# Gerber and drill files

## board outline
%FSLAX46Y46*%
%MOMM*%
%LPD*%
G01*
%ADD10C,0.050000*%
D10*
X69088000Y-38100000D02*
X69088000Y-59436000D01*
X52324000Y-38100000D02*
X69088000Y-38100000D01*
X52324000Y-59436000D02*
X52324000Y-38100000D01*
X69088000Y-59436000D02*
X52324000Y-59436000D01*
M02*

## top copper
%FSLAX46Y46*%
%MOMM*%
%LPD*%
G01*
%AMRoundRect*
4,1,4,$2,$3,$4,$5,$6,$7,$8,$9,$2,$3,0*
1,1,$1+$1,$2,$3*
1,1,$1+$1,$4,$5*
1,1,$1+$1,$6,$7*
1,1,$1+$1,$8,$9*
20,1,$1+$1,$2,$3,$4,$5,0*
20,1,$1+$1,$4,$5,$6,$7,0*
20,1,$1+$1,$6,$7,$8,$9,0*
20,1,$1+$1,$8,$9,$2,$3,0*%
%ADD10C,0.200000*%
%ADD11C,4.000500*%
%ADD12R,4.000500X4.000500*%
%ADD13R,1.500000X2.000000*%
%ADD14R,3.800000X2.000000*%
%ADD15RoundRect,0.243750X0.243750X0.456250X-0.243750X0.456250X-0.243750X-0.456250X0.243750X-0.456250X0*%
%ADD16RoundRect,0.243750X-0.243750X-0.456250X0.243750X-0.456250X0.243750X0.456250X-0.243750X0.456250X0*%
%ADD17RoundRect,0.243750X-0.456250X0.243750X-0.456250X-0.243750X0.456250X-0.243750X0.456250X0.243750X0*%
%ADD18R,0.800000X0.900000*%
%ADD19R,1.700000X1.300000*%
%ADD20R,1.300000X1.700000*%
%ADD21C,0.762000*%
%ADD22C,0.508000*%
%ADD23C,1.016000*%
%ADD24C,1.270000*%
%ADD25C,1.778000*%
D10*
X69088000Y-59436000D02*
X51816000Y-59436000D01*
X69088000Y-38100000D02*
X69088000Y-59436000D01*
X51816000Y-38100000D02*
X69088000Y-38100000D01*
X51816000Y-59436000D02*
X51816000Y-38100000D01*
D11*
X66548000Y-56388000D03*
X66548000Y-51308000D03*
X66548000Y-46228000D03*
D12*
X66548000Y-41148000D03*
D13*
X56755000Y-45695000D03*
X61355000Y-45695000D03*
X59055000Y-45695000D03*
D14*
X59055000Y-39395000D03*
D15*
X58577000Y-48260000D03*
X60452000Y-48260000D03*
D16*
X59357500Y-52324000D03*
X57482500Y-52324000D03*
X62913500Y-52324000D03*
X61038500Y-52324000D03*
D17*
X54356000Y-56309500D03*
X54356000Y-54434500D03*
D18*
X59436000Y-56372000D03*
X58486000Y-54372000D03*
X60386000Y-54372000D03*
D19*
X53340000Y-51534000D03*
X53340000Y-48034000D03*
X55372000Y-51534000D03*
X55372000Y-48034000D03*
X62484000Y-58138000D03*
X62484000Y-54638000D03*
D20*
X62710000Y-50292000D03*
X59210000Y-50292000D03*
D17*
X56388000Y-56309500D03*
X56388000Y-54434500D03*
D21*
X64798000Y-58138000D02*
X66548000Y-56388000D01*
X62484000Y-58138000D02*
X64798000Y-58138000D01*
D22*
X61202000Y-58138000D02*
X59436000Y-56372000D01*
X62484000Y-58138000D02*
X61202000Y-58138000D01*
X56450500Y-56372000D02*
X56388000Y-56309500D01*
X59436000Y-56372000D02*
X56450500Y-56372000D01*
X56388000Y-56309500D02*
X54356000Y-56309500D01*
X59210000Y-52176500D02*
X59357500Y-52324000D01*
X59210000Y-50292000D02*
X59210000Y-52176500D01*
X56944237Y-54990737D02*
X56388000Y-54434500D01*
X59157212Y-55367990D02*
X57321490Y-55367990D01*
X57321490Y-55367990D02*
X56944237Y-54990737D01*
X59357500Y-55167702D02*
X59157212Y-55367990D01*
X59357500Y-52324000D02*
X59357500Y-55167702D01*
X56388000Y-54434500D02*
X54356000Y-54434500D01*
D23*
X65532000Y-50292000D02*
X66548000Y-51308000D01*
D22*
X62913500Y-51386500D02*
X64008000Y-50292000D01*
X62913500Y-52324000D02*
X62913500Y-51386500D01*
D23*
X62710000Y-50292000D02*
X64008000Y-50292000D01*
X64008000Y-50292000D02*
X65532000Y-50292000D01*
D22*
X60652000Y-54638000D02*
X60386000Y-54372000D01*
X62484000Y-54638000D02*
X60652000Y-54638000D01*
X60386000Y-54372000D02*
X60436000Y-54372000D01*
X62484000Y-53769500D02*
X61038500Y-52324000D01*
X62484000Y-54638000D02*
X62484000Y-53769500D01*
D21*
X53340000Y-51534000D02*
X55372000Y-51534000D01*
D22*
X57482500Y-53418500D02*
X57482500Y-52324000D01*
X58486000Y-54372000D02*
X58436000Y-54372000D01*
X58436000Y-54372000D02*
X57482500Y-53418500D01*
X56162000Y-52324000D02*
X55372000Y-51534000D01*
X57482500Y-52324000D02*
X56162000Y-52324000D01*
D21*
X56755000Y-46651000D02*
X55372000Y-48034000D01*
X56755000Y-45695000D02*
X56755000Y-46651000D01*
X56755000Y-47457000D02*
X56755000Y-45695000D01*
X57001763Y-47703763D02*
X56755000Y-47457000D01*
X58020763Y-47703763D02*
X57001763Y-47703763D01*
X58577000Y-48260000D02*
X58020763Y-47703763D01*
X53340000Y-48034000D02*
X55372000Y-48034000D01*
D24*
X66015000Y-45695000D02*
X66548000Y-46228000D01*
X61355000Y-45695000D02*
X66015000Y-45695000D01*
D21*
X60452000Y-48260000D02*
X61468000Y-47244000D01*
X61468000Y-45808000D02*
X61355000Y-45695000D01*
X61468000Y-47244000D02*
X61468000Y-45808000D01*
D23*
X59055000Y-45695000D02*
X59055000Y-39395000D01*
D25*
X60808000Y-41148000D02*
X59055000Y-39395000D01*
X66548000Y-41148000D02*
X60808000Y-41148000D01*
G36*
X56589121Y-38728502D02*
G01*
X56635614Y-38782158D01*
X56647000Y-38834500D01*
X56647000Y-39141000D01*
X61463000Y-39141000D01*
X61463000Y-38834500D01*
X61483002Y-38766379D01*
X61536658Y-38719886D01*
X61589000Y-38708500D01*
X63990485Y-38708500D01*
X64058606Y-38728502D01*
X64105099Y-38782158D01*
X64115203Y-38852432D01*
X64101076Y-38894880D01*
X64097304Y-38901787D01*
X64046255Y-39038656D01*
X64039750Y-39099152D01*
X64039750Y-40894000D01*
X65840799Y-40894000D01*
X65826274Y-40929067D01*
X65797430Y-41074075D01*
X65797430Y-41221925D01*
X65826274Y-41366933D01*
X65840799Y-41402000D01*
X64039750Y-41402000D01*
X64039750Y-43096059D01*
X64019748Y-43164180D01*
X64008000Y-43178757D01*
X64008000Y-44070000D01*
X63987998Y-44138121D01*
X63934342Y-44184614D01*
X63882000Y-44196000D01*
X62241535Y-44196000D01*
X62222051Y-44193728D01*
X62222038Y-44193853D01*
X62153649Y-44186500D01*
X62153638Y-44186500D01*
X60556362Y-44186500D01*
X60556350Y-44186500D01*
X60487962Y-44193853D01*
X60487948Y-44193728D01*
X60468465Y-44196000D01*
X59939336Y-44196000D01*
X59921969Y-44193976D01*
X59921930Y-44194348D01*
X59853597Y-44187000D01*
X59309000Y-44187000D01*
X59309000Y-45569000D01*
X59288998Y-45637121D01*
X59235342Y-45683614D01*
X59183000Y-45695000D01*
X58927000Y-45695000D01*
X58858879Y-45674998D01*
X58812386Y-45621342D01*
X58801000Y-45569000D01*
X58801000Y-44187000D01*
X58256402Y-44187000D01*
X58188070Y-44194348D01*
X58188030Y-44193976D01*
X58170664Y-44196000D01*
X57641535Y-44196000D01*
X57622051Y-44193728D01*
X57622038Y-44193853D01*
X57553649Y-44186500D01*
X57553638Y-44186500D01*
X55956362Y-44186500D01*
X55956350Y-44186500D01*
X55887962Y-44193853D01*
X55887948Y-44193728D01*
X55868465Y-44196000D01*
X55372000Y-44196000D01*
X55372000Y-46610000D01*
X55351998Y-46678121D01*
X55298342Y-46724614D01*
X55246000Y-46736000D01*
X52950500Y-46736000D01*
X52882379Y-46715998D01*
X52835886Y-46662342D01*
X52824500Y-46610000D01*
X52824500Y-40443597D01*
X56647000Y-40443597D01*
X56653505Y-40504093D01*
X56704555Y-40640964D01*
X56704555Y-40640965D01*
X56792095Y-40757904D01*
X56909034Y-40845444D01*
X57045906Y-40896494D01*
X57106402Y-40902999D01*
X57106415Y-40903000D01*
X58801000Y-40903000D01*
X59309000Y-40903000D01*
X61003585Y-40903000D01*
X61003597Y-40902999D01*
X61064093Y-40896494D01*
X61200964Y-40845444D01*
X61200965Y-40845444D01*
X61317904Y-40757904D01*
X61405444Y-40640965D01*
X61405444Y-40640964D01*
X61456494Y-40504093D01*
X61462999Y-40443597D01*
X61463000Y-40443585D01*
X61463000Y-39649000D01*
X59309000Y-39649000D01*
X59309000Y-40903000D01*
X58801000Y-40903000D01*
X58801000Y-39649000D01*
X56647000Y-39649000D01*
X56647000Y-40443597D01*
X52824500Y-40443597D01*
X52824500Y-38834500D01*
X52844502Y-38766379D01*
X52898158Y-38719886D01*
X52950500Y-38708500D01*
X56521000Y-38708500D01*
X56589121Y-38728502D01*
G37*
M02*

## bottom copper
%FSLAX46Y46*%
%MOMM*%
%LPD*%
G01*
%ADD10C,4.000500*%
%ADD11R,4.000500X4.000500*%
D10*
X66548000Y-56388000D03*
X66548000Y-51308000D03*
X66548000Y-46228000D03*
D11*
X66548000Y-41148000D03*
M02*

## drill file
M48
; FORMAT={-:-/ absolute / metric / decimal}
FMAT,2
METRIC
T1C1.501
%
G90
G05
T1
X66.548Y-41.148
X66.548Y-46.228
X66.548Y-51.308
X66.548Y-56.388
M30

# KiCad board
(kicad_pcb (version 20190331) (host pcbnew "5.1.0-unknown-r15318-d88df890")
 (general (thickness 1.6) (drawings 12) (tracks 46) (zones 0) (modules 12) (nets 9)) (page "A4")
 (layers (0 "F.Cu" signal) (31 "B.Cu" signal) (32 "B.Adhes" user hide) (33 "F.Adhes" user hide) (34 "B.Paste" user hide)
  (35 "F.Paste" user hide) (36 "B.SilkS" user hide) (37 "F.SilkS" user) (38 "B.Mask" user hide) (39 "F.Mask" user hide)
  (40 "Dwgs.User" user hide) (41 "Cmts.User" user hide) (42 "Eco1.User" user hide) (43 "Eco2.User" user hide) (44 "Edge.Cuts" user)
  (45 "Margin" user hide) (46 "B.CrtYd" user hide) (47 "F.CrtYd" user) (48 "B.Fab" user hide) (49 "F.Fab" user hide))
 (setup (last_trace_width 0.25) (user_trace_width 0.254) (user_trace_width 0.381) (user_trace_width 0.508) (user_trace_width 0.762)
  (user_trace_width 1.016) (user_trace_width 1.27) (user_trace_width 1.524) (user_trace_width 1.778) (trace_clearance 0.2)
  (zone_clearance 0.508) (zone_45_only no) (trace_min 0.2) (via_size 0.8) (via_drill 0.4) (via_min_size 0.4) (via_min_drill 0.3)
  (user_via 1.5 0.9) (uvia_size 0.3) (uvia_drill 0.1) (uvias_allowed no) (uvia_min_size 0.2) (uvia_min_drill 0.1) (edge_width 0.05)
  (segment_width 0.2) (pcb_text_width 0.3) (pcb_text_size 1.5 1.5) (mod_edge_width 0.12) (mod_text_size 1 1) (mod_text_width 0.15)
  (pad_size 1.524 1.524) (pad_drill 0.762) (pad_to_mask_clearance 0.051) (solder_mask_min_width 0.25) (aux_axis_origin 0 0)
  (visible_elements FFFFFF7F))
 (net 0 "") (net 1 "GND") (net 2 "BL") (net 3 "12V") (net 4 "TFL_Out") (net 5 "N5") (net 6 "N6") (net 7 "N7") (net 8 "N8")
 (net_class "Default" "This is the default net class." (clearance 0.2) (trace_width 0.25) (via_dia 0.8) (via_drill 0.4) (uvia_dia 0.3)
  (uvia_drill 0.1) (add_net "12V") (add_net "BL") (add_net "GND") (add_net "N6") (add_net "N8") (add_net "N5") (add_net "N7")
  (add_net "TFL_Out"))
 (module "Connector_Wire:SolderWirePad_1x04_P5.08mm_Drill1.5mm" (layer "F.Cu") (at 66.548 41.148 270)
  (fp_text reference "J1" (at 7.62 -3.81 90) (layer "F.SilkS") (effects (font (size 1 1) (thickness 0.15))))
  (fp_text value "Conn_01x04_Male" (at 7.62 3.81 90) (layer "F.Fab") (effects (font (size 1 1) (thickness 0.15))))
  (pad "4" thru_hole circle (at 15.24 0 270) (size 4.0005 4.0005) (drill 1.50114) (layers *.Cu *.Mask) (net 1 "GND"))
  (pad "3" thru_hole circle (at 10.16 0 270) (size 4.0005 4.0005) (drill 1.50114) (layers *.Cu *.Mask) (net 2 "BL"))
  (pad "2" thru_hole circle (at 5.08 0 270) (size 4.0005 4.0005) (drill 1.50114) (layers *.Cu *.Mask) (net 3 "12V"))
  (pad "1" thru_hole rect (at 0 0 270) (size 4.0005 4.0005) (drill 1.50114) (layers *.Cu *.Mask) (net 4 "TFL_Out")))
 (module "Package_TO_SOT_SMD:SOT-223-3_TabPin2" (layer "F.Cu") (at 59.055 42.545 90)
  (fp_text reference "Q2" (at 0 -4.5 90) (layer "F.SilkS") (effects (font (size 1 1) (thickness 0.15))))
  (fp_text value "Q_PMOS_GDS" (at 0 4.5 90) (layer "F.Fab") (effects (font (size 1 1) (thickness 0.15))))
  (pad "1" smd rect (at -3.15 -2.3 90) (size 2 1.5) (layers "F.Cu" "F.Paste" "F.Mask") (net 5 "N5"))
  (pad "3" smd rect (at -3.15 2.3 90) (size 2 1.5) (layers "F.Cu" "F.Paste" "F.Mask") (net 3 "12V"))
  (pad "2" smd rect (at -3.15 0 90) (size 2 1.5) (layers "F.Cu" "F.Paste" "F.Mask") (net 4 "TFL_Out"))
  (pad "2" smd rect (at 3.15 0 90) (size 2 3.8) (layers "F.Cu" "F.Paste" "F.Mask") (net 4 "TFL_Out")))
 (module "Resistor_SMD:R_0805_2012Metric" (layer "F.Cu") (at 59.5145 48.26 180)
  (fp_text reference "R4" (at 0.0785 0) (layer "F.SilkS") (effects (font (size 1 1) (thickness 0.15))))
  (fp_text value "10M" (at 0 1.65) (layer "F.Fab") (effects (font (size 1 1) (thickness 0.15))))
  (pad "2" smd roundrect (at 0.9375 0 180) (size 0.975 1.4) (layers "F.Cu" "F.Paste" "F.Mask") (roundrect_rratio 0.25) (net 5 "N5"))
  (pad "1" smd roundrect (at -0.9375 0 180) (size 0.975 1.4) (layers "F.Cu" "F.Paste" "F.Mask") (roundrect_rratio 0.25) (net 3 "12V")))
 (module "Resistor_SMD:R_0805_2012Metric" (layer "F.Cu") (at 58.42 52.324)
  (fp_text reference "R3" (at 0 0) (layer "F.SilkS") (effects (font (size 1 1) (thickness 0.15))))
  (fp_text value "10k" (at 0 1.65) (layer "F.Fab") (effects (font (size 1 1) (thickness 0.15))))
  (pad "2" smd roundrect (at 0.9375 0) (size 0.975 1.4) (layers "F.Cu" "F.Paste" "F.Mask") (roundrect_rratio 0.25) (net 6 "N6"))
  (pad "1" smd roundrect (at -0.9375 0) (size 0.975 1.4) (layers "F.Cu" "F.Paste" "F.Mask") (roundrect_rratio 0.25) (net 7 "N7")))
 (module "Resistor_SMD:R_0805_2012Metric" (layer "F.Cu") (at 61.976 52.324)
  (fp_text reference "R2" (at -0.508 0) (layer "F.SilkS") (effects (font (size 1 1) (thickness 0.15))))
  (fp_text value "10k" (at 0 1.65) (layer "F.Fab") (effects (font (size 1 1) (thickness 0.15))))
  (pad "2" smd roundrect (at 0.9375 0) (size 0.975 1.4) (layers "F.Cu" "F.Paste" "F.Mask") (roundrect_rratio 0.25) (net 2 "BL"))
  (pad "1" smd roundrect (at -0.9375 0) (size 0.975 1.4) (layers "F.Cu" "F.Paste" "F.Mask") (roundrect_rratio 0.25) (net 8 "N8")))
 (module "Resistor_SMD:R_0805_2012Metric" (layer "F.Cu") (at 54.356 55.372 270)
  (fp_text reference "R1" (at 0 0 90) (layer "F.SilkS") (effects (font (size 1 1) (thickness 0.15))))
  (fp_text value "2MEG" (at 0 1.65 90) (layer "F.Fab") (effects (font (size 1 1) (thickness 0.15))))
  (pad "2" smd roundrect (at 0.9375 0 270) (size 0.975 1.4) (layers "F.Cu" "F.Paste" "F.Mask") (roundrect_rratio 0.25) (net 1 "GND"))
  (pad "1" smd roundrect (at -0.9375 0 270) (size 0.975 1.4) (layers "F.Cu" "F.Paste" "F.Mask") (roundrect_rratio 0.25) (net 6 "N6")))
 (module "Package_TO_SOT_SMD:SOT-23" (layer "F.Cu") (at 59.436 55.372 270)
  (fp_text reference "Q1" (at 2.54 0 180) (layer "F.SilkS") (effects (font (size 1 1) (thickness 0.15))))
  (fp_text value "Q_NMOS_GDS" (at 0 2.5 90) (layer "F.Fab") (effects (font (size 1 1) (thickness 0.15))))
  (pad "3" smd rect (at 1 0 270) (size 0.9 0.8) (layers "F.Cu" "F.Paste" "F.Mask") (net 1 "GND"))
  (pad "2" smd rect (at -1 0.95 270) (size 0.9 0.8) (layers "F.Cu" "F.Paste" "F.Mask") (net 7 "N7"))
  (pad "1" smd rect (at -1 -0.95 270) (size 0.9 0.8) (layers "F.Cu" "F.Paste" "F.Mask") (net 8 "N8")))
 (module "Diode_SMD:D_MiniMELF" (layer "F.Cu") (at 53.34 49.784 270)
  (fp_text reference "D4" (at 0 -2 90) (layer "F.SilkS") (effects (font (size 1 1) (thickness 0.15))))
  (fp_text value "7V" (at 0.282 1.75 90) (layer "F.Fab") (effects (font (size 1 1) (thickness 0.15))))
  (pad "2" smd rect (at 1.75 0 270) (size 1.3 1.7) (layers "F.Cu" "F.Paste" "F.Mask") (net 7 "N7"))
  (pad "1" smd rect (at -1.75 0 270) (size 1.3 1.7) (layers "F.Cu" "F.Paste" "F.Mask") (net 5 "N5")))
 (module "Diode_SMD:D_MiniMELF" (layer "F.Cu") (at 55.372 49.784 270)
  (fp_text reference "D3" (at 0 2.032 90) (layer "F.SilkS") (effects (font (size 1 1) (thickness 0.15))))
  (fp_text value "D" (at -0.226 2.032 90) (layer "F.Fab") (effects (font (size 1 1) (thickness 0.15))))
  (pad "2" smd rect (at 1.75 0 270) (size 1.3 1.7) (layers "F.Cu" "F.Paste" "F.Mask") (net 7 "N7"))
  (pad "1" smd rect (at -1.75 0 270) (size 1.3 1.7) (layers "F.Cu" "F.Paste" "F.Mask") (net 5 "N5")))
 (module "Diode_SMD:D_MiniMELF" (layer "F.Cu") (at 62.484 56.388 270)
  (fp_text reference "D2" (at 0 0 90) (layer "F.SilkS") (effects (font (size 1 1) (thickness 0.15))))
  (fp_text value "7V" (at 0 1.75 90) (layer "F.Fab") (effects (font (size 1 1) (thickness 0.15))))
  (pad "2" smd rect (at 1.75 0 270) (size 1.3 1.7) (layers "F.Cu" "F.Paste" "F.Mask") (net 1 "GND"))
  (pad "1" smd rect (at -1.75 0 270) (size 1.3 1.7) (layers "F.Cu" "F.Paste" "F.Mask") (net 8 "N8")))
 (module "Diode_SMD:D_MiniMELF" (layer "F.Cu") (at 60.96 50.292)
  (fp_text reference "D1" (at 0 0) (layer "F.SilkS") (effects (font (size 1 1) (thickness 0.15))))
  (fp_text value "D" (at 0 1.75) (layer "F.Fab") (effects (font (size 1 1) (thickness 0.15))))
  (pad "2" smd rect (at 1.75 0) (size 1.3 1.7) (layers "F.Cu" "F.Paste" "F.Mask") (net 2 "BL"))
  (pad "1" smd rect (at -1.75 0) (size 1.3 1.7) (layers "F.Cu" "F.Paste" "F.Mask") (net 6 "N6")))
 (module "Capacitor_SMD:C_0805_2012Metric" (layer "F.Cu") (at 56.388 55.372 270)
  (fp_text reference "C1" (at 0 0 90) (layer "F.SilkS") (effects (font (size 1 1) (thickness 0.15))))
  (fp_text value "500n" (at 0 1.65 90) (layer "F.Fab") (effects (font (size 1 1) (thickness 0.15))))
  (pad "2" smd roundrect (at 0.9375 0 270) (size 0.975 1.4) (layers "F.Cu" "F.Paste" "F.Mask") (roundrect_rratio 0.25) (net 1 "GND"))
  (pad "1" smd roundrect (at -0.9375 0 270) (size 0.975 1.4) (layers "F.Cu" "F.Paste" "F.Mask") (roundrect_rratio 0.25) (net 6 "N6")))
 (gr_line (start 69.088 59.436) (end 51.816 59.436) (layer "F.Cu") (width 0.2))
 (gr_line (start 69.088 38.1) (end 69.088 59.436) (layer "F.Cu") (width 0.2))
 (gr_line (start 51.816 38.1) (end 69.088 38.1) (layer "F.Cu") (width 0.2))
 (gr_line (start 51.816 59.436) (end 51.816 38.1) (layer "F.Cu") (width 0.2))
 (gr_line (start 69.088 38.1) (end 69.088 59.436) (layer "Edge.Cuts") (width 0.05))
 (gr_line (start 52.324 38.1) (end 69.088 38.1) (layer "Edge.Cuts") (width 0.05))
 (gr_line (start 52.324 59.436) (end 52.324 38.1) (layer "Edge.Cuts") (width 0.05))
 (gr_line (start 69.088 59.436) (end 52.324 59.436) (layer "Edge.Cuts") (width 0.05))
 (segment (start 64.798 58.138) (end 66.548 56.388) (width 0.762) (layer "F.Cu") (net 1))
 (segment (start 62.484 58.138) (end 64.798 58.138) (width 0.762) (layer "F.Cu") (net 1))
 (segment (start 61.202 58.138) (end 59.436 56.372) (width 0.508) (layer "F.Cu") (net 1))
 (segment (start 62.484 58.138) (end 61.202 58.138) (width 0.508) (layer "F.Cu") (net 1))
 (segment (start 56.4505 56.372) (end 56.388 56.3095) (width 0.508) (layer "F.Cu") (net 1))
 (segment (start 59.436 56.372) (end 56.4505 56.372) (width 0.508) (layer "F.Cu") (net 1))
 (segment (start 56.388 56.3095) (end 54.356 56.3095) (width 0.508) (layer "F.Cu") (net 1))
 (segment (start 59.21 52.1765) (end 59.3575 52.324) (width 0.508) (layer "F.Cu") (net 6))
 (segment (start 59.21 50.292) (end 59.21 52.1765) (width 0.508) (layer "F.Cu") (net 6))
 (segment (start 56.944237 54.990737) (end 56.388 54.4345) (width 0.508) (layer "F.Cu") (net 6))
 (segment (start 59.157212 55.36799) (end 57.32149 55.36799) (width 0.508) (layer "F.Cu") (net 6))
 (segment (start 57.32149 55.36799) (end 56.944237 54.990737) (width 0.508) (layer "F.Cu") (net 6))
 (segment (start 59.3575 55.167702) (end 59.157212 55.36799) (width 0.508) (layer "F.Cu") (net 6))
 (segment (start 59.3575 52.324) (end 59.3575 55.167702) (width 0.508) (layer "F.Cu") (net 6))
 (segment (start 56.388 54.4345) (end 54.356 54.4345) (width 0.508) (layer "F.Cu") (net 6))
 (segment (start 65.532 50.292) (end 66.548 51.308) (width 1.016) (layer "F.Cu") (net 2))
 (segment (start 62.9135 51.3865) (end 64.008 50.292) (width 0.508) (layer "F.Cu") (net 2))
 (segment (start 62.9135 52.324) (end 62.9135 51.3865) (width 0.508) (layer "F.Cu") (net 2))
 (segment (start 62.71 50.292) (end 64.008 50.292) (width 1.016) (layer "F.Cu") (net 2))
 (segment (start 64.008 50.292) (end 65.532 50.292) (width 1.016) (layer "F.Cu") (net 2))
 (segment (start 60.652 54.638) (end 60.386 54.372) (width 0.508) (layer "F.Cu") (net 8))
 (segment (start 62.484 54.638) (end 60.652 54.638) (width 0.508) (layer "F.Cu") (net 8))
 (segment (start 60.386 54.372) (end 60.436 54.372) (width 0.508) (layer "F.Cu") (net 8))
 (segment (start 62.484 53.7695) (end 61.0385 52.324) (width 0.508) (layer "F.Cu") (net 8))
 (segment (start 62.484 54.638) (end 62.484 53.7695) (width 0.508) (layer "F.Cu") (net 8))
 (segment (start 53.34 51.534) (end 55.372 51.534) (width 0.762) (layer "F.Cu") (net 7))
 (segment (start 57.4825 53.4185) (end 57.4825 52.324) (width 0.508) (layer "F.Cu") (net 7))
 (segment (start 58.486 54.372) (end 58.436 54.372) (width 0.508) (layer "F.Cu") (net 7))
 (segment (start 58.436 54.372) (end 57.4825 53.4185) (width 0.508) (layer "F.Cu") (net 7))
 (segment (start 56.162 52.324) (end 55.372 51.534) (width 0.508) (layer "F.Cu") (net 7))
 (segment (start 57.4825 52.324) (end 56.162 52.324) (width 0.508) (layer "F.Cu") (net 7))
 (segment (start 56.755 46.651) (end 55.372 48.034) (width 0.762) (layer "F.Cu") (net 5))
 (segment (start 56.755 45.695) (end 56.755 46.651) (width 0.762) (layer "F.Cu") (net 5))
 (segment (start 56.755 47.457) (end 56.755 45.695) (width 0.762) (layer "F.Cu") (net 5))
 (segment (start 57.001763 47.703763) (end 56.755 47.457) (width 0.762) (layer "F.Cu") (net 5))
 (segment (start 58.020763 47.703763) (end 57.001763 47.703763) (width 0.762) (layer "F.Cu") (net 5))
 (segment (start 58.577 48.26) (end 58.020763 47.703763) (width 0.762) (layer "F.Cu") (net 5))
 (segment (start 53.34 48.034) (end 55.372 48.034) (width 0.762) (layer "F.Cu") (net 5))
 (segment (start 66.015 45.695) (end 66.548 46.228) (width 1.27) (layer "F.Cu") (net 3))
 (segment (start 61.355 45.695) (end 66.015 45.695) (width 1.27) (layer "F.Cu") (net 3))
 (segment (start 60.452 48.26) (end 61.468 47.244) (width 0.762) (layer "F.Cu") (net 3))
 (segment (start 61.468 45.808) (end 61.355 45.695) (width 0.762) (layer "F.Cu") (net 3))
 (segment (start 61.468 47.244) (end 61.468 45.808) (width 0.762) (layer "F.Cu") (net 3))
 (segment (start 59.055 45.695) (end 59.055 39.395) (width 1.016) (layer "F.Cu") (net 4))
 (segment (start 60.808 41.148) (end 59.055 39.395) (width 1.778) (layer "F.Cu") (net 4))
 (segment (start 66.548 41.148) (end 60.808 41.148) (width 1.778) (layer "F.Cu") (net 4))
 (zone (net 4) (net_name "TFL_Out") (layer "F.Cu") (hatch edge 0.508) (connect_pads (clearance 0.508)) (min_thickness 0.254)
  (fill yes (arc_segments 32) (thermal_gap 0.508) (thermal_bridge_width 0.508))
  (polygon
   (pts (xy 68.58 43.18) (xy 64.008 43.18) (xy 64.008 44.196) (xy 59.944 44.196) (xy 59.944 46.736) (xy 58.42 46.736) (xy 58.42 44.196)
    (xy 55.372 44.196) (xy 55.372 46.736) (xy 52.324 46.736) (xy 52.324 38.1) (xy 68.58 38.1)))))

